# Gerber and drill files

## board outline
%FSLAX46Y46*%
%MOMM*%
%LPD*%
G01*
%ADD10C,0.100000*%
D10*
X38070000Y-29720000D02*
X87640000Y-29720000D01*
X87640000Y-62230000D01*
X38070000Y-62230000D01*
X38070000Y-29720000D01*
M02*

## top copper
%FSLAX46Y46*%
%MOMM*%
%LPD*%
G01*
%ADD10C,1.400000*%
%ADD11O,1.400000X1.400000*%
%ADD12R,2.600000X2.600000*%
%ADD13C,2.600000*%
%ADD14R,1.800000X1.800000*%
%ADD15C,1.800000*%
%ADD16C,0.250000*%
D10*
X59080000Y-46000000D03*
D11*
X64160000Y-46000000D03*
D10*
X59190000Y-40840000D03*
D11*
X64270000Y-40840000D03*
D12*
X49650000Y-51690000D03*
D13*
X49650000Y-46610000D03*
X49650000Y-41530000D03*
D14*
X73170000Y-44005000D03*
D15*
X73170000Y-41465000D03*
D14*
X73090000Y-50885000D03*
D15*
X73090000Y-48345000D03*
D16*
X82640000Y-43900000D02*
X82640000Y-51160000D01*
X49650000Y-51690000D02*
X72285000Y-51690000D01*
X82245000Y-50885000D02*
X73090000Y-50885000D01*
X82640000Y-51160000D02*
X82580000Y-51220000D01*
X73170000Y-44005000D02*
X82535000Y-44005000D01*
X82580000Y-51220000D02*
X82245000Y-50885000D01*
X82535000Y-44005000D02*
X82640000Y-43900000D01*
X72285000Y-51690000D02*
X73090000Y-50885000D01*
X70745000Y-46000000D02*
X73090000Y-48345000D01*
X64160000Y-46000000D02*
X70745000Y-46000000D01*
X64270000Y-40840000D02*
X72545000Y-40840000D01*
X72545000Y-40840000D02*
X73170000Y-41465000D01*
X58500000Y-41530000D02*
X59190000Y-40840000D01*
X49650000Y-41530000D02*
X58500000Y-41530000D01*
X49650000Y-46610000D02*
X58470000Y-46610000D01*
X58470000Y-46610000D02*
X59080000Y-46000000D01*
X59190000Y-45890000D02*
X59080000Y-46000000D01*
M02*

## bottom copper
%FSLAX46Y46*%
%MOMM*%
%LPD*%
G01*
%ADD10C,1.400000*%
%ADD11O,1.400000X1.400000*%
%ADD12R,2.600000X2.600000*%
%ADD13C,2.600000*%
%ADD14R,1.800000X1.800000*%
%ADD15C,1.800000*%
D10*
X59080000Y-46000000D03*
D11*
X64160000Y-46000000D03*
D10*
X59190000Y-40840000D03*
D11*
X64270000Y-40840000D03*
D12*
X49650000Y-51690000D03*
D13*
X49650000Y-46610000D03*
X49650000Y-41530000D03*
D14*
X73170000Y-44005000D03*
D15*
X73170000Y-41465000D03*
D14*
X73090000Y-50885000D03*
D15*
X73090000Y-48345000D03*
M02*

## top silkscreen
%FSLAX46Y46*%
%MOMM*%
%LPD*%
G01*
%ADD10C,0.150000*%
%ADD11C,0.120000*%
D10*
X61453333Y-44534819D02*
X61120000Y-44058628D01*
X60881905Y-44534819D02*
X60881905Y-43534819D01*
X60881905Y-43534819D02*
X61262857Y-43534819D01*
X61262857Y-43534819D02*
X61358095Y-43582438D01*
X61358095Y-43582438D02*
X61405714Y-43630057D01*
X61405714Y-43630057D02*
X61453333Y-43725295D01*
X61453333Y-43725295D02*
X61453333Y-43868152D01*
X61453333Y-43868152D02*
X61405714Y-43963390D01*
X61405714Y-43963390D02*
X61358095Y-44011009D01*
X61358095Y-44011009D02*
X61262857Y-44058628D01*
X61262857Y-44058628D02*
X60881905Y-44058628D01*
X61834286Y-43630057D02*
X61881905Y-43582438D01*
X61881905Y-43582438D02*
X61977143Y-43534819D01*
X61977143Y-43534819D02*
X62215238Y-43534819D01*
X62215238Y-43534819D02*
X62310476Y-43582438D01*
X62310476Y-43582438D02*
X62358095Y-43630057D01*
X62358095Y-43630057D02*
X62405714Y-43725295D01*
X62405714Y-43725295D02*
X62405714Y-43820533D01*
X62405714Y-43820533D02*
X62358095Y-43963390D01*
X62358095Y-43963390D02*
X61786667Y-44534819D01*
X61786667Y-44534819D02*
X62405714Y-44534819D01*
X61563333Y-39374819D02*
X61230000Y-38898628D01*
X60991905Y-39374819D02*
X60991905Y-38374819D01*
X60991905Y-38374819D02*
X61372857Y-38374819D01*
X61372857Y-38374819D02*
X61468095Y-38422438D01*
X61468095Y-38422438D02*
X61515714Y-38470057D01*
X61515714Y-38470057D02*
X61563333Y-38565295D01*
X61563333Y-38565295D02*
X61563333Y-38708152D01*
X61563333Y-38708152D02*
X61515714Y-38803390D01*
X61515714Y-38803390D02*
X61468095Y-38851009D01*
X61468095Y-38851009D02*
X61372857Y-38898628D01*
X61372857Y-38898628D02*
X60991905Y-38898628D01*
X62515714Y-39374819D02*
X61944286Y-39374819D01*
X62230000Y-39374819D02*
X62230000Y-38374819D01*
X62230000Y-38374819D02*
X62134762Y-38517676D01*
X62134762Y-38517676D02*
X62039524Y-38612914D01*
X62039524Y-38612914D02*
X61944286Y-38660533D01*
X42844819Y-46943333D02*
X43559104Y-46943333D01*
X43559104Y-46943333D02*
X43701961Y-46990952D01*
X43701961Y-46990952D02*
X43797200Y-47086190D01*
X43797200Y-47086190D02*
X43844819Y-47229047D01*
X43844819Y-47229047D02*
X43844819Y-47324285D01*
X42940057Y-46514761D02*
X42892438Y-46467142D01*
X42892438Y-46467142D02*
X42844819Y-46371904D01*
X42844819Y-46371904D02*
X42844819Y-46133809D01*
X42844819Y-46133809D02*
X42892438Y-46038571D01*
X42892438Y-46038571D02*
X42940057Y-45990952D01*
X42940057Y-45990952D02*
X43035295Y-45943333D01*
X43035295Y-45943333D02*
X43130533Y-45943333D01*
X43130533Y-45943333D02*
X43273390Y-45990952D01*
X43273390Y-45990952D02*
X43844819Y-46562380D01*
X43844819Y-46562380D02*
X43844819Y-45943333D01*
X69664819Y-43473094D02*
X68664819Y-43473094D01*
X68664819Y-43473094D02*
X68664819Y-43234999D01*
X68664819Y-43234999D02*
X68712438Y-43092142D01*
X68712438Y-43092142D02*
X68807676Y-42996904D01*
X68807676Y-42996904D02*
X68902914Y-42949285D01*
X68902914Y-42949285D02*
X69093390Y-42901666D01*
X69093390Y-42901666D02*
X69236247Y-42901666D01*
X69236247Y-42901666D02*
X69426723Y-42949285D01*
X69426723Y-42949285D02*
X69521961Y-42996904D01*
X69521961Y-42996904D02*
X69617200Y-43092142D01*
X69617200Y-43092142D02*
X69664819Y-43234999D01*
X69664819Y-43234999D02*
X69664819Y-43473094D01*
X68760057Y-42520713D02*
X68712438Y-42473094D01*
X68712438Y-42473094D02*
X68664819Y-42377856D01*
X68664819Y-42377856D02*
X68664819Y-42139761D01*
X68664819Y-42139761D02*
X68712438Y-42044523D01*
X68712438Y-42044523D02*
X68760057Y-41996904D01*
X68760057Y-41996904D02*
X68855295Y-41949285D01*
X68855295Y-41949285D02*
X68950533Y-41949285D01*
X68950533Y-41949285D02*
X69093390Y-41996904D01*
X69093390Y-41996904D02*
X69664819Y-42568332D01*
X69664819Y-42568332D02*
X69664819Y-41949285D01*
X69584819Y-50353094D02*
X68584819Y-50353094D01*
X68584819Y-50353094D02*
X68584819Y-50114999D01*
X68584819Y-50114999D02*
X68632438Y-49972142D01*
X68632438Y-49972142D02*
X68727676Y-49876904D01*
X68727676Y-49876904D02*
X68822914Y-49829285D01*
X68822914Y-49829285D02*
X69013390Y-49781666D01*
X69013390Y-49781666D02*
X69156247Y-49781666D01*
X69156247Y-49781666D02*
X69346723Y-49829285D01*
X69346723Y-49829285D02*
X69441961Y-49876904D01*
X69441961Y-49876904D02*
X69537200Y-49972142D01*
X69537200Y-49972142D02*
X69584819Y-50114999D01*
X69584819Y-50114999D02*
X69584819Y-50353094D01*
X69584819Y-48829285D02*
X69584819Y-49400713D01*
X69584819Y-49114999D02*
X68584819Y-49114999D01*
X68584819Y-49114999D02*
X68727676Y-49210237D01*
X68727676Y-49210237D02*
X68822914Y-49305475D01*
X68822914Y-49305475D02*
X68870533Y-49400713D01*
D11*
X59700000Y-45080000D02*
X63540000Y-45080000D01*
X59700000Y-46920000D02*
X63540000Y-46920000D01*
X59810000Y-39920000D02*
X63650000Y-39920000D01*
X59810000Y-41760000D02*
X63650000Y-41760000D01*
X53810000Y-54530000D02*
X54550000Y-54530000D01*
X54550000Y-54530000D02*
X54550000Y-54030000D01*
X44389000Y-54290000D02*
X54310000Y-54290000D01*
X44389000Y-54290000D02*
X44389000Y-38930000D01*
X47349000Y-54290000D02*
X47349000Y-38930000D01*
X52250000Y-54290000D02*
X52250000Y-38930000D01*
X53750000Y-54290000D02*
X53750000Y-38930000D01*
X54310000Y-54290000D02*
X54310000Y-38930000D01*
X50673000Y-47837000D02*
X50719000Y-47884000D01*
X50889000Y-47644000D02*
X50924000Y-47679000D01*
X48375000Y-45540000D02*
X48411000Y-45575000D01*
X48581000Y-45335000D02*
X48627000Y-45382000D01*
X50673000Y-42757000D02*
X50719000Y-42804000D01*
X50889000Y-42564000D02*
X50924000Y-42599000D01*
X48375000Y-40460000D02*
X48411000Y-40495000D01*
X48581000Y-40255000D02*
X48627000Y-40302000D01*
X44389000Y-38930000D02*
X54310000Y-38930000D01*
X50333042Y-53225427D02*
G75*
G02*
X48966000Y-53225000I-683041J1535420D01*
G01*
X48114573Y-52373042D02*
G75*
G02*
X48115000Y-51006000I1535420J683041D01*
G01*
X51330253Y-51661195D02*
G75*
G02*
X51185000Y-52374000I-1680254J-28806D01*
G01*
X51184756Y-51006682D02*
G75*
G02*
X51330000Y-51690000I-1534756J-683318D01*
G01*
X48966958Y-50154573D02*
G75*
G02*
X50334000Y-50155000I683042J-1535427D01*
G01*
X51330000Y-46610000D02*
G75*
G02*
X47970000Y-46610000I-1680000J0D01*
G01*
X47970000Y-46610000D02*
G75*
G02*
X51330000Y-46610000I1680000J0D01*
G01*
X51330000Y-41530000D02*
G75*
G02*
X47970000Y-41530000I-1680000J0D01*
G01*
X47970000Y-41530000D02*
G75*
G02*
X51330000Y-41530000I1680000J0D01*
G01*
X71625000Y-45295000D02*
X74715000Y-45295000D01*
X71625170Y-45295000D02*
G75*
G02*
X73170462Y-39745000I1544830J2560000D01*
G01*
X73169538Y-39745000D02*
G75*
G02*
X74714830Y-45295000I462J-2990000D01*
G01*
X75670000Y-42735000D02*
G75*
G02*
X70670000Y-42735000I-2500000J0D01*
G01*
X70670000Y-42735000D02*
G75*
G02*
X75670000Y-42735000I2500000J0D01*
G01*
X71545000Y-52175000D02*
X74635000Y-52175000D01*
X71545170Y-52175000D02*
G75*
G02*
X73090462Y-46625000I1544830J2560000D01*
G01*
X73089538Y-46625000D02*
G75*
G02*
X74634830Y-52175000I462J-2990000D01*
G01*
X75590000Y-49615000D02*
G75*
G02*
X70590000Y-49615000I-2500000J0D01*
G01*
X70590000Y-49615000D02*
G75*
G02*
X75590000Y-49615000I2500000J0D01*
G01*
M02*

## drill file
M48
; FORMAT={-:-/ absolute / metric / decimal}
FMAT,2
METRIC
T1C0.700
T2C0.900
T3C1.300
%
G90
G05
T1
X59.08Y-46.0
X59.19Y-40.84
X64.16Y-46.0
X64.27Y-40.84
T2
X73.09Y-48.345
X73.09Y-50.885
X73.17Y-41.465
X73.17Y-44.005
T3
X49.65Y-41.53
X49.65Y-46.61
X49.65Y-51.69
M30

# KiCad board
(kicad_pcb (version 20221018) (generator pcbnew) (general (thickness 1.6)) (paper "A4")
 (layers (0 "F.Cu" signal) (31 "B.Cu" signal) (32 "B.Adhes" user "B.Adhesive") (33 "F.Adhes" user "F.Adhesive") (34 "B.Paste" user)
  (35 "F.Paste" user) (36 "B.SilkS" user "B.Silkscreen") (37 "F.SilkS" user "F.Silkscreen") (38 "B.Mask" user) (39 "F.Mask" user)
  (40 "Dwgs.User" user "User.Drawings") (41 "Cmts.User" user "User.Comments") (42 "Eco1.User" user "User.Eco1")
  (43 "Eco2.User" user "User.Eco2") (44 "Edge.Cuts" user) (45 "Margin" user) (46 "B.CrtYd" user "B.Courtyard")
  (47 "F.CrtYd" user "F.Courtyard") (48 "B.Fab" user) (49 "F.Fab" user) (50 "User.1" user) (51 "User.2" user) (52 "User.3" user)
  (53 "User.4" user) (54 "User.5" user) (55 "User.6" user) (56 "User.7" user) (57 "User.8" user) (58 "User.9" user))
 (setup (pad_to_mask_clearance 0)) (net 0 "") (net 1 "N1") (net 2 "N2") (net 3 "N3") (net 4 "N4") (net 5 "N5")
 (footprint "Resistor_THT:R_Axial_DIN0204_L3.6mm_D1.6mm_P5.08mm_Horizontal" (layer "F.Cu") (at 59.08 46)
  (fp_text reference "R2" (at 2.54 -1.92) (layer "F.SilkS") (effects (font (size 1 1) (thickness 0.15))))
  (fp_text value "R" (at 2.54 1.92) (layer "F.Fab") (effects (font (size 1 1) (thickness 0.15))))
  (fp_line (start 0.62 -0.92) (end 4.46 -0.92) (stroke (width 0.12) (type solid)) (layer "F.SilkS"))
  (fp_line (start 0.62 0.92) (end 4.46 0.92) (stroke (width 0.12) (type solid)) (layer "F.SilkS"))
  (pad "1" thru_hole circle (at 0 0) (size 1.4 1.4) (drill 0.7) (layers "*.Cu" "*.Mask") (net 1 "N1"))
  (pad "2" thru_hole oval (at 5.08 0) (size 1.4 1.4) (drill 0.7) (layers "*.Cu" "*.Mask") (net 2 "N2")))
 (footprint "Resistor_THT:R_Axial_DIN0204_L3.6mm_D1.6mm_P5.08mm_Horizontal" (layer "F.Cu") (at 59.19 40.84)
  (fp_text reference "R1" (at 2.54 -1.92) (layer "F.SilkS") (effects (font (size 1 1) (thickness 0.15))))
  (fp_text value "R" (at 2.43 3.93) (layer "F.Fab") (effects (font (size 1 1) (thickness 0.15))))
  (fp_line (start 0.62 -0.92) (end 4.46 -0.92) (stroke (width 0.12) (type solid)) (layer "F.SilkS"))
  (fp_line (start 0.62 0.92) (end 4.46 0.92) (stroke (width 0.12) (type solid)) (layer "F.SilkS"))
  (pad "1" thru_hole circle (at 0 0) (size 1.4 1.4) (drill 0.7) (layers "*.Cu" "*.Mask") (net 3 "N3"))
  (pad "2" thru_hole oval (at 5.08 0) (size 1.4 1.4) (drill 0.7) (layers "*.Cu" "*.Mask") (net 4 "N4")))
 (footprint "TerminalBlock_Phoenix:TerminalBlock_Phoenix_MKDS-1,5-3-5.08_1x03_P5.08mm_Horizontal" (layer "F.Cu") (at 49.65 51.69 90)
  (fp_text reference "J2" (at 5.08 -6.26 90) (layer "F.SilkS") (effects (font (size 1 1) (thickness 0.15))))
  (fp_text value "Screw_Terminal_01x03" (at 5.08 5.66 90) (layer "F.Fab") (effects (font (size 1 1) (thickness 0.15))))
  (fp_line (start -2.84 4.16) (end -2.84 4.9) (stroke (width 0.12) (type solid)) (layer "F.SilkS"))
  (fp_line (start -2.84 4.9) (end -2.34 4.9) (stroke (width 0.12) (type solid)) (layer "F.SilkS"))
  (fp_line (start -2.6 -5.261) (end -2.6 4.66) (stroke (width 0.12) (type solid)) (layer "F.SilkS"))
  (fp_line (start -2.6 -5.261) (end 12.76 -5.261) (stroke (width 0.12) (type solid)) (layer "F.SilkS"))
  (fp_line (start -2.6 -2.301) (end 12.76 -2.301) (stroke (width 0.12) (type solid)) (layer "F.SilkS"))
  (fp_line (start -2.6 2.6) (end 12.76 2.6) (stroke (width 0.12) (type solid)) (layer "F.SilkS"))
  (fp_line (start -2.6 4.1) (end 12.76 4.1) (stroke (width 0.12) (type solid)) (layer "F.SilkS"))
  (fp_line (start -2.6 4.66) (end 12.76 4.66) (stroke (width 0.12) (type solid)) (layer "F.SilkS"))
  (fp_line (start 3.853 1.023) (end 3.806 1.069) (stroke (width 0.12) (type solid)) (layer "F.SilkS"))
  (fp_line (start 4.046 1.239) (end 4.011 1.274) (stroke (width 0.12) (type solid)) (layer "F.SilkS"))
  (fp_line (start 6.15 -1.275) (end 6.115 -1.239) (stroke (width 0.12) (type solid)) (layer "F.SilkS"))
  (fp_line (start 6.355 -1.069) (end 6.308 -1.023) (stroke (width 0.12) (type solid)) (layer "F.SilkS"))
  (fp_line (start 8.933 1.023) (end 8.886 1.069) (stroke (width 0.12) (type solid)) (layer "F.SilkS"))
  (fp_line (start 9.126 1.239) (end 9.091 1.274) (stroke (width 0.12) (type solid)) (layer "F.SilkS"))
  (fp_line (start 11.23 -1.275) (end 11.195 -1.239) (stroke (width 0.12) (type solid)) (layer "F.SilkS"))
  (fp_line (start 11.435 -1.069) (end 11.388 -1.023) (stroke (width 0.12) (type solid)) (layer "F.SilkS"))
  (fp_line (start 12.76 -5.261) (end 12.76 4.66) (stroke (width 0.12) (type solid)) (layer "F.SilkS"))
  (fp_arc (start -1.535427 0.683042) (mid -1.680501 -0.000524) (end -1.535 -0.684) (stroke (width 0.12) (type solid)) (layer "F.SilkS"))
  (fp_arc (start -0.683042 -1.535427) (mid 0.000524 -1.680501) (end 0.684 -1.535) (stroke (width 0.12) (type solid)) (layer "F.SilkS"))
  (fp_arc (start 0.028805 1.680253) (mid -0.335551 1.646659) (end -0.684 1.535) (stroke (width 0.12) (type solid)) (layer "F.SilkS"))
  (fp_arc (start 0.683318 1.534756) (mid 0.349292 1.643288) (end 0 1.68) (stroke (width 0.12) (type solid)) (layer "F.SilkS"))
  (fp_arc (start 1.535427 -0.683042) (mid 1.680501 0.000524) (end 1.535 0.684) (stroke (width 0.12) (type solid)) (layer "F.SilkS"))
  (fp_circle (center 5.08 0) (end 6.76 0) (stroke (width 0.12) (type solid)) (fill none) (layer "F.SilkS"))
  (fp_circle (center 10.16 0) (end 11.84 0) (stroke (width 0.12) (type solid)) (fill none) (layer "F.SilkS"))
  (pad "1" thru_hole rect (at 0 0 90) (size 2.6 2.6) (drill 1.3) (layers "*.Cu" "*.Mask") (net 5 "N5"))
  (pad "2" thru_hole circle (at 5.08 0 90) (size 2.6 2.6) (drill 1.3) (layers "*.Cu" "*.Mask") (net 1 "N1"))
  (pad "3" thru_hole circle (at 10.16 0 90) (size 2.6 2.6) (drill 1.3) (layers "*.Cu" "*.Mask") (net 3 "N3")))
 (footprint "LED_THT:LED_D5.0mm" (layer "F.Cu") (at 73.17 44.005 90)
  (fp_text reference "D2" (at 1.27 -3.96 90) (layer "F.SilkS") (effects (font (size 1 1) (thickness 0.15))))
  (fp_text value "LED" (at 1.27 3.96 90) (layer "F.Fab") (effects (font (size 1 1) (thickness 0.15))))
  (fp_line (start -1.29 -1.545) (end -1.29 1.545) (stroke (width 0.12) (type solid)) (layer "F.SilkS"))
  (fp_arc (start -1.29 -1.54483) (mid 2.072002 -2.880433) (end 4.26 0.000462) (stroke (width 0.12) (type solid)) (layer "F.SilkS"))
  (fp_arc (start 4.26 -0.000462) (mid 2.072002 2.880433) (end -1.29 1.54483) (stroke (width 0.12) (type solid)) (layer "F.SilkS"))
  (fp_circle (center 1.27 0) (end 3.77 0) (stroke (width 0.12) (type solid)) (fill none) (layer "F.SilkS"))
  (pad "1" thru_hole rect (at 0 0 90) (size 1.8 1.8) (drill 0.9) (layers "*.Cu" "*.Mask") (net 5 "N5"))
  (pad "2" thru_hole circle (at 2.54 0 90) (size 1.8 1.8) (drill 0.9) (layers "*.Cu" "*.Mask") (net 4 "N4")))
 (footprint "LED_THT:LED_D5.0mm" (layer "F.Cu") (at 73.09 50.885 90)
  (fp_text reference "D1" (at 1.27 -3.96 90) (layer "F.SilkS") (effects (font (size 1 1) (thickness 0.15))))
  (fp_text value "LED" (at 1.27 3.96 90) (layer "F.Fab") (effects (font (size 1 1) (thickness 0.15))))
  (fp_line (start -1.29 -1.545) (end -1.29 1.545) (stroke (width 0.12) (type solid)) (layer "F.SilkS"))
  (fp_arc (start -1.29 -1.54483) (mid 2.072002 -2.880433) (end 4.26 0.000462) (stroke (width 0.12) (type solid)) (layer "F.SilkS"))
  (fp_arc (start 4.26 -0.000462) (mid 2.072002 2.880433) (end -1.29 1.54483) (stroke (width 0.12) (type solid)) (layer "F.SilkS"))
  (fp_circle (center 1.27 0) (end 3.77 0) (stroke (width 0.12) (type solid)) (fill none) (layer "F.SilkS"))
  (pad "1" thru_hole rect (at 0 0 90) (size 1.8 1.8) (drill 0.9) (layers "*.Cu" "*.Mask") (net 5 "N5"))
  (pad "2" thru_hole circle (at 2.54 0 90) (size 1.8 1.8) (drill 0.9) (layers "*.Cu" "*.Mask") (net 2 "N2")))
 (gr_rect (start 38.07 29.72) (end 87.64 62.23) (stroke (width 0.1) (type default)) (fill none) (layer "Edge.Cuts"))
 (segment (start 82.64 43.9) (end 82.64 51.16) (width 0.25) (layer "F.Cu") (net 5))
 (segment (start 49.65 51.69) (end 72.285 51.69) (width 0.25) (layer "F.Cu") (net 5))
 (segment (start 82.245 50.885) (end 73.09 50.885) (width 0.25) (layer "F.Cu") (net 5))
 (segment (start 82.64 51.16) (end 82.58 51.22) (width 0.25) (layer "F.Cu") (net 5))
 (segment (start 73.17 44.005) (end 82.535 44.005) (width 0.25) (layer "F.Cu") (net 5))
 (segment (start 82.58 51.22) (end 82.245 50.885) (width 0.25) (layer "F.Cu") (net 5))
 (segment (start 82.535 44.005) (end 82.64 43.9) (width 0.25) (layer "F.Cu") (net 5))
 (segment (start 72.285 51.69) (end 73.09 50.885) (width 0.25) (layer "F.Cu") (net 5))
 (segment (start 70.745 46) (end 73.09 48.345) (width 0.25) (layer "F.Cu") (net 2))
 (segment (start 64.16 46) (end 70.745 46) (width 0.25) (layer "F.Cu") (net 2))
 (segment (start 64.27 40.84) (end 72.545 40.84) (width 0.25) (layer "F.Cu") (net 4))
 (segment (start 72.545 40.84) (end 73.17 41.465) (width 0.25) (layer "F.Cu") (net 4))
 (segment (start 58.5 41.53) (end 59.19 40.84) (width 0.25) (layer "F.Cu") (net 3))
 (segment (start 49.65 41.53) (end 58.5 41.53) (width 0.25) (layer "F.Cu") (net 3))
 (segment (start 49.65 46.61) (end 58.47 46.61) (width 0.25) (layer "F.Cu") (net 1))
 (segment (start 58.47 46.61) (end 59.08 46) (width 0.25) (layer "F.Cu") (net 1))
 (segment (start 59.19 45.89) (end 59.08 46) (width 0.25) (layer "F.Cu") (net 1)))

